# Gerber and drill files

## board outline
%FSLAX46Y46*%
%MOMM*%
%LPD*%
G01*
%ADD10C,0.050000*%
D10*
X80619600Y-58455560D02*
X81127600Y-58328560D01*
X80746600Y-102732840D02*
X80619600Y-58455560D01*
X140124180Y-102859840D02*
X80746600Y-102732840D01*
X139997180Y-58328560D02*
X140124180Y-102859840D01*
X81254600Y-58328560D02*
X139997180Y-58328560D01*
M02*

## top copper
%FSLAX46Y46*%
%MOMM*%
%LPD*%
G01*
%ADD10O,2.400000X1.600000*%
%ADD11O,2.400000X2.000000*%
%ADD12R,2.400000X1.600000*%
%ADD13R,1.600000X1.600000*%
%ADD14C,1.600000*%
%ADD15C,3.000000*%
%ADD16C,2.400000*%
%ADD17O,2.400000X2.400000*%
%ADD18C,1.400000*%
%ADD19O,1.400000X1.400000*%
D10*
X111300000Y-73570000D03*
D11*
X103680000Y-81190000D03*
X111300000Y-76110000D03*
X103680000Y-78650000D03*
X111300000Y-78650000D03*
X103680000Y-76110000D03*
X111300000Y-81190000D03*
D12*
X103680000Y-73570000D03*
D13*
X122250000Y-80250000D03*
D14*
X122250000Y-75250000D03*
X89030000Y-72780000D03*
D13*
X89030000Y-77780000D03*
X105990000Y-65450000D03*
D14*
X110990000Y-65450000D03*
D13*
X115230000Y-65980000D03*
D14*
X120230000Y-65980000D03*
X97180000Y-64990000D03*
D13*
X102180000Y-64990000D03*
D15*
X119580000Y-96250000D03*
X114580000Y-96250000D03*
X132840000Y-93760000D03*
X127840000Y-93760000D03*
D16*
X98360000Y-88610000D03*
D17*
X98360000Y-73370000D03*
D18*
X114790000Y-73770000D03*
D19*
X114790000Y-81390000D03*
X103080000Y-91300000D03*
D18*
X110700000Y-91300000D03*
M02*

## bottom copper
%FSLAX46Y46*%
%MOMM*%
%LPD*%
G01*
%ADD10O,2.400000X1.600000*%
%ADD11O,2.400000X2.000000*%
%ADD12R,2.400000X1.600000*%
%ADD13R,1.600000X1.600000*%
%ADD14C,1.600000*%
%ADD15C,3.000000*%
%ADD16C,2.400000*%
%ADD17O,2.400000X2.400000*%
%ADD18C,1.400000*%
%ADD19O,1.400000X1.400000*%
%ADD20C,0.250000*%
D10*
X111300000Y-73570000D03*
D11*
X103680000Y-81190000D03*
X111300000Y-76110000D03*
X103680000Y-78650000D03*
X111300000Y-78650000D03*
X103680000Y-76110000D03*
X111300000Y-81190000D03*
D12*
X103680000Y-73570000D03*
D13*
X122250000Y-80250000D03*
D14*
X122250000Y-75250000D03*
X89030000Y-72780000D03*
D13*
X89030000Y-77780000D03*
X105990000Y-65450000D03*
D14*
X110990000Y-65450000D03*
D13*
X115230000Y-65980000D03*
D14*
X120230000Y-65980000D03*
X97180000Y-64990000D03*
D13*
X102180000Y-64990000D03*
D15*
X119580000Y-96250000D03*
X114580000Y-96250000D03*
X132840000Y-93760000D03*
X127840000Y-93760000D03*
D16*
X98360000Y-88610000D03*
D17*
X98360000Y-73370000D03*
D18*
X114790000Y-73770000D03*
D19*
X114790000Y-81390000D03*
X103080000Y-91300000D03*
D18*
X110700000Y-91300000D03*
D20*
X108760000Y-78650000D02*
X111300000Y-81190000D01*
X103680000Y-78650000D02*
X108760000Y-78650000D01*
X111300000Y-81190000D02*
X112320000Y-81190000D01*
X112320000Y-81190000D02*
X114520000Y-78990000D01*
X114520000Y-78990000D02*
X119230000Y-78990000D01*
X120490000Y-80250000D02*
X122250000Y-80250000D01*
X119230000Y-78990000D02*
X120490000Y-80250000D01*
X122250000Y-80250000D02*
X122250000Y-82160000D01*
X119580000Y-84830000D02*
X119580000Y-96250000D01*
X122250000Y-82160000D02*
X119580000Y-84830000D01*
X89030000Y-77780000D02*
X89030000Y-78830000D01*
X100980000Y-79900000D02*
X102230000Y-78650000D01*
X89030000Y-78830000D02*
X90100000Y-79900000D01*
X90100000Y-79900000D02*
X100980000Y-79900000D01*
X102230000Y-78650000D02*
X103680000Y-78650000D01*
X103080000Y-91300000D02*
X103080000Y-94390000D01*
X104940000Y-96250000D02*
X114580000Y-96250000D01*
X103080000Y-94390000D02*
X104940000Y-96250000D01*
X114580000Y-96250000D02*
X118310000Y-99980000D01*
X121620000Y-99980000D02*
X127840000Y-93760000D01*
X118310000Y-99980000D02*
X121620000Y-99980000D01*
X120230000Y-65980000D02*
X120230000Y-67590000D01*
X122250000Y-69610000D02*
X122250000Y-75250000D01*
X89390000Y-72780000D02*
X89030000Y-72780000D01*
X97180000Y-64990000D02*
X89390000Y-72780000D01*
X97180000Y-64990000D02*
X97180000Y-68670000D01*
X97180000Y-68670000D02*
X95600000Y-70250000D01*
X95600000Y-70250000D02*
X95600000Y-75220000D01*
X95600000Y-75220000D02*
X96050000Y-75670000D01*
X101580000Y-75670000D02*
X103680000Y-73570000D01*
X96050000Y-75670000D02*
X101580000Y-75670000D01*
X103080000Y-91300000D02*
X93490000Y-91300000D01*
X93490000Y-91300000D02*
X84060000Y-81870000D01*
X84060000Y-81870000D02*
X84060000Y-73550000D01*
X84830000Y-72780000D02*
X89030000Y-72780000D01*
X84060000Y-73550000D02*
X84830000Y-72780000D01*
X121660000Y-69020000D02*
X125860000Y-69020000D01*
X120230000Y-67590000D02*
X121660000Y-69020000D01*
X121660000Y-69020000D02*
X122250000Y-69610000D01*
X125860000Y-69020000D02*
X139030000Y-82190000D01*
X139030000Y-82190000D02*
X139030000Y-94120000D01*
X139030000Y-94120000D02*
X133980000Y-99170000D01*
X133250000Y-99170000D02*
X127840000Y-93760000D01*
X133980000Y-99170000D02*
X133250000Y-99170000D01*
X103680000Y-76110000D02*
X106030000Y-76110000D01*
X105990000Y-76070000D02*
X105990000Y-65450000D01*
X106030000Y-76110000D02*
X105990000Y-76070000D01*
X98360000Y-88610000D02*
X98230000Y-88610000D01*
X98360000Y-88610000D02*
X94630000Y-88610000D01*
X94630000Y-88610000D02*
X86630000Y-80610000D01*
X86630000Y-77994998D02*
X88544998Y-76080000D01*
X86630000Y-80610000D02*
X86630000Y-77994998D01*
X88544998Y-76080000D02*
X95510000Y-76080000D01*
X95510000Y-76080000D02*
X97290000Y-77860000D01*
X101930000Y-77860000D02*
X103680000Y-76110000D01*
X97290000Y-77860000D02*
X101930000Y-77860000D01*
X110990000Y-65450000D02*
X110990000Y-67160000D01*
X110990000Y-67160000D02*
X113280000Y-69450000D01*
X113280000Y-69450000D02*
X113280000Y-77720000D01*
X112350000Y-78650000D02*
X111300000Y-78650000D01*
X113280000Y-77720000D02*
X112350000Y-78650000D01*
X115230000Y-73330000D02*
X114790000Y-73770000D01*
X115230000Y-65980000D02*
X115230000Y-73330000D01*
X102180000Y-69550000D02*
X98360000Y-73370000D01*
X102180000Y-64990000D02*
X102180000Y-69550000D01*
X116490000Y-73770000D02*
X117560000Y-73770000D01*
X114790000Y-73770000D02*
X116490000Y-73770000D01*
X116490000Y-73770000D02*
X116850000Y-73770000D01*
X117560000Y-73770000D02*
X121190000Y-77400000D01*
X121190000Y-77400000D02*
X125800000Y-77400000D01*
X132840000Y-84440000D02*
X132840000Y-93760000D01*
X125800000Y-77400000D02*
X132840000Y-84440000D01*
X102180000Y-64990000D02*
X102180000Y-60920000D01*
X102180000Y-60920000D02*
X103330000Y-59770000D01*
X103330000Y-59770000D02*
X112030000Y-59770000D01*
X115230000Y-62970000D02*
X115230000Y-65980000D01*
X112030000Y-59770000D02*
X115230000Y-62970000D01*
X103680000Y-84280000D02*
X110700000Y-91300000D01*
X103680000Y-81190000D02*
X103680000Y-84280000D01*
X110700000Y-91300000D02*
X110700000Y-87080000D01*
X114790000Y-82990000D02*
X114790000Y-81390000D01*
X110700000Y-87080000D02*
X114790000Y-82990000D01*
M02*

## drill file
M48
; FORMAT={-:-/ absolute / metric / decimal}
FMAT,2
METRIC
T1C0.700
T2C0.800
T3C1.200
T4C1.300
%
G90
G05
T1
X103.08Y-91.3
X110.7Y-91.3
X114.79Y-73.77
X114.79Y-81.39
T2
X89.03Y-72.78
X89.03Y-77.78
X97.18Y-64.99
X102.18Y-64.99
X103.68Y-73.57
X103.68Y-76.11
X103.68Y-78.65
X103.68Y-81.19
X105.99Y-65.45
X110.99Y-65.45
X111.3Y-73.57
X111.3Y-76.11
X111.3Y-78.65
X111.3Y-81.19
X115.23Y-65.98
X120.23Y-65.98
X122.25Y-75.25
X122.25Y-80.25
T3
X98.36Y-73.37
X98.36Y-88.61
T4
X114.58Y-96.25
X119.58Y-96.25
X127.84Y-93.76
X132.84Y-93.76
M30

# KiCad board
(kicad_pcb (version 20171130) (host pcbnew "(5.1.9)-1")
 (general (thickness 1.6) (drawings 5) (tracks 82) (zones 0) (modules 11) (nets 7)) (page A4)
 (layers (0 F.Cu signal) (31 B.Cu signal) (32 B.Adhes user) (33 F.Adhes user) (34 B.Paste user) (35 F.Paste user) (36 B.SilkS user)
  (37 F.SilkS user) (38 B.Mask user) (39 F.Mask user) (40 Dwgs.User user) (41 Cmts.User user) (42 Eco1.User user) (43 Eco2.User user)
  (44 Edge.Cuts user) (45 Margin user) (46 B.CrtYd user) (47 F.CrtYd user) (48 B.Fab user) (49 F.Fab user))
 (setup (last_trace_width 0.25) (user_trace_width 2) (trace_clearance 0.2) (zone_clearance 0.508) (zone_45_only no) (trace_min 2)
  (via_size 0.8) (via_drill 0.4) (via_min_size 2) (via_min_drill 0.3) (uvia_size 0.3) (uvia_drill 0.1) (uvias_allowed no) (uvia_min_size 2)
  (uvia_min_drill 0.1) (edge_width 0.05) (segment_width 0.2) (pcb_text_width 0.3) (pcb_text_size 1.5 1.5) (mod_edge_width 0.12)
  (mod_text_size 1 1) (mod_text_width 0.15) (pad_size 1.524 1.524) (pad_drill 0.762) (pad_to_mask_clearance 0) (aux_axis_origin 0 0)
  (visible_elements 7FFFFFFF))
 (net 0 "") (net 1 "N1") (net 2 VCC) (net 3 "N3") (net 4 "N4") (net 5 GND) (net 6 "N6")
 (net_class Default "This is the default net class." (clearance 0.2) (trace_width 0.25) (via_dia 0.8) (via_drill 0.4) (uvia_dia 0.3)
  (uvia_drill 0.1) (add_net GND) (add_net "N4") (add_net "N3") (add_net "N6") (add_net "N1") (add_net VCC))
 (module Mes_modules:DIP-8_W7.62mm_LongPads (layer F.Cu) (at 103.68 73.57)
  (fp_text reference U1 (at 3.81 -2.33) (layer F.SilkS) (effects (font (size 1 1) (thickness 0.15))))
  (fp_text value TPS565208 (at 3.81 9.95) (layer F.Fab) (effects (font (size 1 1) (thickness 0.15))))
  (pad 8 thru_hole oval (at 7.62 0) (size 2.4 1.6) (drill 0.8) (layers *.Cu *.Mask))
  (pad 4 thru_hole oval (at 0 7.62) (size 2.4 2) (drill 0.8) (layers *.Cu *.Mask) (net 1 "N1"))
  (pad 7 thru_hole oval (at 7.62 2.54) (size 2.4 2) (drill 0.8) (layers *.Cu *.Mask))
  (pad 3 thru_hole oval (at 0 5.08) (size 2.4 2) (drill 0.8) (layers *.Cu *.Mask) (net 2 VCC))
  (pad 6 thru_hole oval (at 7.62 5.08) (size 2.4 2) (drill 0.8) (layers *.Cu *.Mask) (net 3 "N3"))
  (pad 2 thru_hole oval (at 0 2.54) (size 2.4 2) (drill 0.8) (layers *.Cu *.Mask) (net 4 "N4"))
  (pad 5 thru_hole oval (at 7.62 7.62) (size 2.4 2) (drill 0.8) (layers *.Cu *.Mask) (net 2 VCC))
  (pad 1 thru_hole rect (at 0 0) (size 2.4 1.6) (drill 0.8) (layers *.Cu *.Mask) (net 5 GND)))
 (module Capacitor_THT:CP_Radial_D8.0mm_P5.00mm (layer F.Cu) (at 122.25 80.25 90)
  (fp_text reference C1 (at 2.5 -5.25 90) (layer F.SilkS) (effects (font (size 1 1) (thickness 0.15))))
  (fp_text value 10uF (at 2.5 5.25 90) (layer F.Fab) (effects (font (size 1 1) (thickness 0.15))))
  (pad 1 thru_hole rect (at 0 0 90) (size 1.6 1.6) (drill 0.8) (layers *.Cu *.Mask) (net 2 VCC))
  (pad 2 thru_hole circle (at 5 0 90) (size 1.6 1.6) (drill 0.8) (layers *.Cu *.Mask) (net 5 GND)))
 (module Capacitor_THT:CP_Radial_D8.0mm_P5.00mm (layer F.Cu) (at 89.03 77.78 90)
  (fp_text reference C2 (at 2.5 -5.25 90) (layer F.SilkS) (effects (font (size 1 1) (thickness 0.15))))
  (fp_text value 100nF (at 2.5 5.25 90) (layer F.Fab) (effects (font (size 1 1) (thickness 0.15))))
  (pad 2 thru_hole circle (at 5 0 90) (size 1.6 1.6) (drill 0.8) (layers *.Cu *.Mask) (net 5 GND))
  (pad 1 thru_hole rect (at 0 0 90) (size 1.6 1.6) (drill 0.8) (layers *.Cu *.Mask) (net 2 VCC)))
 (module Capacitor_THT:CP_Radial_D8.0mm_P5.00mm (layer F.Cu) (at 105.99 65.45)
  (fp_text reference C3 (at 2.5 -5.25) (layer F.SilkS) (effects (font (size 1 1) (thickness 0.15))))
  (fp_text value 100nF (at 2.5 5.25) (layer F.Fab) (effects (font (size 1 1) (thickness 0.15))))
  (pad 1 thru_hole rect (at 0 0) (size 1.6 1.6) (drill 0.8) (layers *.Cu *.Mask) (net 4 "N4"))
  (pad 2 thru_hole circle (at 5 0) (size 1.6 1.6) (drill 0.8) (layers *.Cu *.Mask) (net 3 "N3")))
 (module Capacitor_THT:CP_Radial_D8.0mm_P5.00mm (layer F.Cu) (at 115.23 65.98)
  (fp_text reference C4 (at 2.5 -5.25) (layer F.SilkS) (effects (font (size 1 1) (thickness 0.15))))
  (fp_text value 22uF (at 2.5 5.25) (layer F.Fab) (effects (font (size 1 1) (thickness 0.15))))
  (pad 1 thru_hole rect (at 0 0) (size 1.6 1.6) (drill 0.8) (layers *.Cu *.Mask) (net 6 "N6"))
  (pad 2 thru_hole circle (at 5 0) (size 1.6 1.6) (drill 0.8) (layers *.Cu *.Mask) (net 5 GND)))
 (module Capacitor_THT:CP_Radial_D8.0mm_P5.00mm (layer F.Cu) (at 102.18 64.99 180)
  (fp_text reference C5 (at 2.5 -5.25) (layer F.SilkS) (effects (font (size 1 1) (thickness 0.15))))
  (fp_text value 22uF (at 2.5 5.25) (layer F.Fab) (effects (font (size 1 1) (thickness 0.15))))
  (pad 2 thru_hole circle (at 5 0 180) (size 1.6 1.6) (drill 0.8) (layers *.Cu *.Mask) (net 5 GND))
  (pad 1 thru_hole rect (at 0 0 180) (size 1.6 1.6) (drill 0.8) (layers *.Cu *.Mask) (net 6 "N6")))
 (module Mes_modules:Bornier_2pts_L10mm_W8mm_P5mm (layer F.Cu) (at 119.58 96.25 180)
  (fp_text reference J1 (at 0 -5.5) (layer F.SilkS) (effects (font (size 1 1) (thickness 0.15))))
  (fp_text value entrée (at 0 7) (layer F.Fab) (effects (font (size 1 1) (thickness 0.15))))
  (pad 1 thru_hole circle (at 0 0 180) (size 3 3) (drill 1.3) (layers *.Cu *.Mask) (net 2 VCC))
  (pad 2 thru_hole circle (at 5 0 180) (size 3 3) (drill 1.3) (layers *.Cu *.Mask) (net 5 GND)))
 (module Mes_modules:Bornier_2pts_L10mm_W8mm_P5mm (layer F.Cu) (at 127.84 93.76)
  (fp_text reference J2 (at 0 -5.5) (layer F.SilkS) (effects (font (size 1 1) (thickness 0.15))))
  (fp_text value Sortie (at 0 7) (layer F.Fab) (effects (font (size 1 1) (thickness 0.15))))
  (pad 2 thru_hole circle (at 5 0) (size 3 3) (drill 1.3) (layers *.Cu *.Mask) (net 6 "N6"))
  (pad 1 thru_hole circle (at 0 0) (size 3 3) (drill 1.3) (layers *.Cu *.Mask) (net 5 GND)))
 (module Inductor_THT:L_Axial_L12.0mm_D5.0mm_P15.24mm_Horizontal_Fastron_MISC (layer F.Cu) (at 98.36 88.61 90)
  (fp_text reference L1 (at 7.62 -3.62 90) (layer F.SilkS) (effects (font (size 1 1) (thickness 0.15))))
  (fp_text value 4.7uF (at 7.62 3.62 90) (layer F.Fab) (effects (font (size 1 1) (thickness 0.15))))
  (pad 1 thru_hole circle (at 0 0 90) (size 2.4 2.4) (drill 1.2) (layers *.Cu *.Mask) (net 4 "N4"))
  (pad 2 thru_hole oval (at 15.24 0 90) (size 2.4 2.4) (drill 1.2) (layers *.Cu *.Mask) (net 6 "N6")))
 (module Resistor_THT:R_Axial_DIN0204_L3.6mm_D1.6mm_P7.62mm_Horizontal (layer F.Cu) (at 114.79 73.77 270)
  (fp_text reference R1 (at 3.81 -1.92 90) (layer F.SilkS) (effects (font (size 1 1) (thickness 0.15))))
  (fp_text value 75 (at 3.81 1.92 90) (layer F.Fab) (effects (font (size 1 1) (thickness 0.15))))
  (pad 1 thru_hole circle (at 0 0 270) (size 1.4 1.4) (drill 0.7) (layers *.Cu *.Mask) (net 6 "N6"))
  (pad 2 thru_hole oval (at 7.62 0 270) (size 1.4 1.4) (drill 0.7) (layers *.Cu *.Mask) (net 1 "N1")))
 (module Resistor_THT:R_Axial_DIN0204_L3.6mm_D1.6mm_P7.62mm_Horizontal (layer F.Cu) (at 110.7 91.3 180)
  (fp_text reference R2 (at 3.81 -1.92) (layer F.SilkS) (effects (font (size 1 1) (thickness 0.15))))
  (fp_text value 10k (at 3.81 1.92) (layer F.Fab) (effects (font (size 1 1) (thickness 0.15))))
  (pad 2 thru_hole oval (at 7.62 0 180) (size 1.4 1.4) (drill 0.7) (layers *.Cu *.Mask) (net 5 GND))
  (pad 1 thru_hole circle (at 0 0 180) (size 1.4 1.4) (drill 0.7) (layers *.Cu *.Mask) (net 1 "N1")))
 (gr_line (start 80.6196 58.45556) (end 81.1276 58.32856) (layer Edge.Cuts) (width 0.05))
 (gr_line (start 80.7466 102.73284) (end 80.6196 58.45556) (layer Edge.Cuts) (width 0.05))
 (gr_line (start 140.12418 102.85984) (end 80.7466 102.73284) (layer Edge.Cuts) (width 0.05))
 (gr_line (start 139.99718 58.32856) (end 140.12418 102.85984) (layer Edge.Cuts) (width 0.05))
 (gr_line (start 81.2546 58.32856) (end 139.99718 58.32856) (layer Edge.Cuts) (width 0.05))
 (segment (start 108.76 78.65) (end 111.3 81.19) (width 0.25) (layer B.Cu) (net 2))
 (segment (start 103.68 78.65) (end 108.76 78.65) (width 0.25) (layer B.Cu) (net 2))
 (segment (start 111.3 81.19) (end 112.32 81.19) (width 0.25) (layer B.Cu) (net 2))
 (segment (start 112.32 81.19) (end 114.52 78.99) (width 0.25) (layer B.Cu) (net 2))
 (segment (start 114.52 78.99) (end 119.23 78.99) (width 0.25) (layer B.Cu) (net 2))
 (segment (start 120.49 80.25) (end 122.25 80.25) (width 0.25) (layer B.Cu) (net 2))
 (segment (start 119.23 78.99) (end 120.49 80.25) (width 0.25) (layer B.Cu) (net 2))
 (segment (start 122.25 80.25) (end 122.25 82.16) (width 0.25) (layer B.Cu) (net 2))
 (segment (start 119.58 84.83) (end 119.58 96.25) (width 0.25) (layer B.Cu) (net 2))
 (segment (start 122.25 82.16) (end 119.58 84.83) (width 0.25) (layer B.Cu) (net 2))
 (segment (start 89.03 77.78) (end 89.03 78.83) (width 0.25) (layer B.Cu) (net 2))
 (segment (start 100.98 79.9) (end 102.23 78.65) (width 0.25) (layer B.Cu) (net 2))
 (segment (start 89.03 78.83) (end 90.1 79.9) (width 0.25) (layer B.Cu) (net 2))
 (segment (start 90.1 79.9) (end 100.98 79.9) (width 0.25) (layer B.Cu) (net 2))
 (segment (start 102.23 78.65) (end 103.68 78.65) (width 0.25) (layer B.Cu) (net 2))
 (segment (start 103.08 91.3) (end 103.08 94.39) (width 0.25) (layer B.Cu) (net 5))
 (segment (start 104.94 96.25) (end 114.58 96.25) (width 0.25) (layer B.Cu) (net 5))
 (segment (start 103.08 94.39) (end 104.94 96.25) (width 0.25) (layer B.Cu) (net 5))
 (segment (start 114.58 96.25) (end 118.31 99.98) (width 0.25) (layer B.Cu) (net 5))
 (segment (start 121.62 99.98) (end 127.84 93.76) (width 0.25) (layer B.Cu) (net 5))
 (segment (start 118.31 99.98) (end 121.62 99.98) (width 0.25) (layer B.Cu) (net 5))
 (segment (start 120.23 65.98) (end 120.23 67.59) (width 0.25) (layer B.Cu) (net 5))
 (segment (start 122.25 69.61) (end 122.25 75.25) (width 0.25) (layer B.Cu) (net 5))
 (segment (start 89.39 72.78) (end 89.03 72.78) (width 0.25) (layer B.Cu) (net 5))
 (segment (start 97.18 64.99) (end 89.39 72.78) (width 0.25) (layer B.Cu) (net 5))
 (segment (start 97.18 64.99) (end 97.18 68.67) (width 0.25) (layer B.Cu) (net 5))
 (segment (start 97.18 68.67) (end 95.6 70.25) (width 0.25) (layer B.Cu) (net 5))
 (segment (start 95.6 70.25) (end 95.6 75.22) (width 0.25) (layer B.Cu) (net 5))
 (segment (start 95.6 75.22) (end 96.05 75.67) (width 0.25) (layer B.Cu) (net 5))
 (segment (start 101.58 75.67) (end 103.68 73.57) (width 0.25) (layer B.Cu) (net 5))
 (segment (start 96.05 75.67) (end 101.58 75.67) (width 0.25) (layer B.Cu) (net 5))
 (segment (start 103.08 91.3) (end 93.49 91.3) (width 0.25) (layer B.Cu) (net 5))
 (segment (start 93.49 91.3) (end 84.06 81.87) (width 0.25) (layer B.Cu) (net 5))
 (segment (start 84.06 81.87) (end 84.06 73.55) (width 0.25) (layer B.Cu) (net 5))
 (segment (start 84.83 72.78) (end 89.03 72.78) (width 0.25) (layer B.Cu) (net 5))
 (segment (start 84.06 73.55) (end 84.83 72.78) (width 0.25) (layer B.Cu) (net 5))
 (segment (start 121.66 69.02) (end 125.86 69.02) (width 0.25) (layer B.Cu) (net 5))
 (segment (start 120.23 67.59) (end 121.66 69.02) (width 0.25) (layer B.Cu) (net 5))
 (segment (start 121.66 69.02) (end 122.25 69.61) (width 0.25) (layer B.Cu) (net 5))
 (segment (start 125.86 69.02) (end 139.03 82.19) (width 0.25) (layer B.Cu) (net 5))
 (segment (start 139.03 82.19) (end 139.03 94.12) (width 0.25) (layer B.Cu) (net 5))
 (segment (start 139.03 94.12) (end 133.98 99.17) (width 0.25) (layer B.Cu) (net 5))
 (segment (start 133.25 99.17) (end 127.84 93.76) (width 0.25) (layer B.Cu) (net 5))
 (segment (start 133.98 99.17) (end 133.25 99.17) (width 0.25) (layer B.Cu) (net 5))
 (segment (start 103.68 76.11) (end 106.03 76.11) (width 0.25) (layer B.Cu) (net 4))
 (segment (start 105.99 76.07) (end 105.99 65.45) (width 0.25) (layer B.Cu) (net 4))
 (segment (start 106.03 76.11) (end 105.99 76.07) (width 0.25) (layer B.Cu) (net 4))
 (segment (start 98.36 88.61) (end 98.23 88.61) (width 0.25) (layer B.Cu) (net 4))
 (segment (start 98.36 88.61) (end 94.63 88.61) (width 0.25) (layer B.Cu) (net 4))
 (segment (start 94.63 88.61) (end 86.63 80.61) (width 0.25) (layer B.Cu) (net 4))
 (segment (start 86.63 77.994998) (end 88.544998 76.08) (width 0.25) (layer B.Cu) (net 4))
 (segment (start 86.63 80.61) (end 86.63 77.994998) (width 0.25) (layer B.Cu) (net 4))
 (segment (start 88.544998 76.08) (end 95.51 76.08) (width 0.25) (layer B.Cu) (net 4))
 (segment (start 95.51 76.08) (end 97.29 77.86) (width 0.25) (layer B.Cu) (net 4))
 (segment (start 101.93 77.86) (end 103.68 76.11) (width 0.25) (layer B.Cu) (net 4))
 (segment (start 97.29 77.86) (end 101.93 77.86) (width 0.25) (layer B.Cu) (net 4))
 (segment (start 110.99 65.45) (end 110.99 67.16) (width 0.25) (layer B.Cu) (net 3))
 (segment (start 110.99 67.16) (end 113.28 69.45) (width 0.25) (layer B.Cu) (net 3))
 (segment (start 113.28 69.45) (end 113.28 77.72) (width 0.25) (layer B.Cu) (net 3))
 (segment (start 112.35 78.65) (end 111.3 78.65) (width 0.25) (layer B.Cu) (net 3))
 (segment (start 113.28 77.72) (end 112.35 78.65) (width 0.25) (layer B.Cu) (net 3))
 (segment (start 115.23 73.33) (end 114.79 73.77) (width 0.25) (layer B.Cu) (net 6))
 (segment (start 115.23 65.98) (end 115.23 73.33) (width 0.25) (layer B.Cu) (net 6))
 (segment (start 102.18 69.55) (end 98.36 73.37) (width 0.25) (layer B.Cu) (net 6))
 (segment (start 102.18 64.99) (end 102.18 69.55) (width 0.25) (layer B.Cu) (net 6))
 (segment (start 116.49 73.77) (end 117.56 73.77) (width 0.25) (layer B.Cu) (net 6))
 (segment (start 114.79 73.77) (end 116.49 73.77) (width 0.25) (layer B.Cu) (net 6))
 (segment (start 116.49 73.77) (end 116.85 73.77) (width 0.25) (layer B.Cu) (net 6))
 (segment (start 117.56 73.77) (end 121.19 77.4) (width 0.25) (layer B.Cu) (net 6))
 (segment (start 121.19 77.4) (end 125.8 77.4) (width 0.25) (layer B.Cu) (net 6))
 (segment (start 132.84 84.44) (end 132.84 93.76) (width 0.25) (layer B.Cu) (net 6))
 (segment (start 125.8 77.4) (end 132.84 84.44) (width 0.25) (layer B.Cu) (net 6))
 (segment (start 102.18 64.99) (end 102.18 60.92) (width 0.25) (layer B.Cu) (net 6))
 (segment (start 102.18 60.92) (end 103.33 59.77) (width 0.25) (layer B.Cu) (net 6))
 (segment (start 103.33 59.77) (end 112.03 59.77) (width 0.25) (layer B.Cu) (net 6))
 (segment (start 115.23 62.97) (end 115.23 65.98) (width 0.25) (layer B.Cu) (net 6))
 (segment (start 112.03 59.77) (end 115.23 62.97) (width 0.25) (layer B.Cu) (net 6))
 (segment (start 103.68 84.28) (end 110.7 91.3) (width 0.25) (layer B.Cu) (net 1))
 (segment (start 103.68 81.19) (end 103.68 84.28) (width 0.25) (layer B.Cu) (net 1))
 (segment (start 110.7 91.3) (end 110.7 87.08) (width 0.25) (layer B.Cu) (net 1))
 (segment (start 114.79 82.99) (end 114.79 81.39) (width 0.25) (layer B.Cu) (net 1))
 (segment (start 110.7 87.08) (end 114.79 82.99) (width 0.25) (layer B.Cu) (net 1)))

